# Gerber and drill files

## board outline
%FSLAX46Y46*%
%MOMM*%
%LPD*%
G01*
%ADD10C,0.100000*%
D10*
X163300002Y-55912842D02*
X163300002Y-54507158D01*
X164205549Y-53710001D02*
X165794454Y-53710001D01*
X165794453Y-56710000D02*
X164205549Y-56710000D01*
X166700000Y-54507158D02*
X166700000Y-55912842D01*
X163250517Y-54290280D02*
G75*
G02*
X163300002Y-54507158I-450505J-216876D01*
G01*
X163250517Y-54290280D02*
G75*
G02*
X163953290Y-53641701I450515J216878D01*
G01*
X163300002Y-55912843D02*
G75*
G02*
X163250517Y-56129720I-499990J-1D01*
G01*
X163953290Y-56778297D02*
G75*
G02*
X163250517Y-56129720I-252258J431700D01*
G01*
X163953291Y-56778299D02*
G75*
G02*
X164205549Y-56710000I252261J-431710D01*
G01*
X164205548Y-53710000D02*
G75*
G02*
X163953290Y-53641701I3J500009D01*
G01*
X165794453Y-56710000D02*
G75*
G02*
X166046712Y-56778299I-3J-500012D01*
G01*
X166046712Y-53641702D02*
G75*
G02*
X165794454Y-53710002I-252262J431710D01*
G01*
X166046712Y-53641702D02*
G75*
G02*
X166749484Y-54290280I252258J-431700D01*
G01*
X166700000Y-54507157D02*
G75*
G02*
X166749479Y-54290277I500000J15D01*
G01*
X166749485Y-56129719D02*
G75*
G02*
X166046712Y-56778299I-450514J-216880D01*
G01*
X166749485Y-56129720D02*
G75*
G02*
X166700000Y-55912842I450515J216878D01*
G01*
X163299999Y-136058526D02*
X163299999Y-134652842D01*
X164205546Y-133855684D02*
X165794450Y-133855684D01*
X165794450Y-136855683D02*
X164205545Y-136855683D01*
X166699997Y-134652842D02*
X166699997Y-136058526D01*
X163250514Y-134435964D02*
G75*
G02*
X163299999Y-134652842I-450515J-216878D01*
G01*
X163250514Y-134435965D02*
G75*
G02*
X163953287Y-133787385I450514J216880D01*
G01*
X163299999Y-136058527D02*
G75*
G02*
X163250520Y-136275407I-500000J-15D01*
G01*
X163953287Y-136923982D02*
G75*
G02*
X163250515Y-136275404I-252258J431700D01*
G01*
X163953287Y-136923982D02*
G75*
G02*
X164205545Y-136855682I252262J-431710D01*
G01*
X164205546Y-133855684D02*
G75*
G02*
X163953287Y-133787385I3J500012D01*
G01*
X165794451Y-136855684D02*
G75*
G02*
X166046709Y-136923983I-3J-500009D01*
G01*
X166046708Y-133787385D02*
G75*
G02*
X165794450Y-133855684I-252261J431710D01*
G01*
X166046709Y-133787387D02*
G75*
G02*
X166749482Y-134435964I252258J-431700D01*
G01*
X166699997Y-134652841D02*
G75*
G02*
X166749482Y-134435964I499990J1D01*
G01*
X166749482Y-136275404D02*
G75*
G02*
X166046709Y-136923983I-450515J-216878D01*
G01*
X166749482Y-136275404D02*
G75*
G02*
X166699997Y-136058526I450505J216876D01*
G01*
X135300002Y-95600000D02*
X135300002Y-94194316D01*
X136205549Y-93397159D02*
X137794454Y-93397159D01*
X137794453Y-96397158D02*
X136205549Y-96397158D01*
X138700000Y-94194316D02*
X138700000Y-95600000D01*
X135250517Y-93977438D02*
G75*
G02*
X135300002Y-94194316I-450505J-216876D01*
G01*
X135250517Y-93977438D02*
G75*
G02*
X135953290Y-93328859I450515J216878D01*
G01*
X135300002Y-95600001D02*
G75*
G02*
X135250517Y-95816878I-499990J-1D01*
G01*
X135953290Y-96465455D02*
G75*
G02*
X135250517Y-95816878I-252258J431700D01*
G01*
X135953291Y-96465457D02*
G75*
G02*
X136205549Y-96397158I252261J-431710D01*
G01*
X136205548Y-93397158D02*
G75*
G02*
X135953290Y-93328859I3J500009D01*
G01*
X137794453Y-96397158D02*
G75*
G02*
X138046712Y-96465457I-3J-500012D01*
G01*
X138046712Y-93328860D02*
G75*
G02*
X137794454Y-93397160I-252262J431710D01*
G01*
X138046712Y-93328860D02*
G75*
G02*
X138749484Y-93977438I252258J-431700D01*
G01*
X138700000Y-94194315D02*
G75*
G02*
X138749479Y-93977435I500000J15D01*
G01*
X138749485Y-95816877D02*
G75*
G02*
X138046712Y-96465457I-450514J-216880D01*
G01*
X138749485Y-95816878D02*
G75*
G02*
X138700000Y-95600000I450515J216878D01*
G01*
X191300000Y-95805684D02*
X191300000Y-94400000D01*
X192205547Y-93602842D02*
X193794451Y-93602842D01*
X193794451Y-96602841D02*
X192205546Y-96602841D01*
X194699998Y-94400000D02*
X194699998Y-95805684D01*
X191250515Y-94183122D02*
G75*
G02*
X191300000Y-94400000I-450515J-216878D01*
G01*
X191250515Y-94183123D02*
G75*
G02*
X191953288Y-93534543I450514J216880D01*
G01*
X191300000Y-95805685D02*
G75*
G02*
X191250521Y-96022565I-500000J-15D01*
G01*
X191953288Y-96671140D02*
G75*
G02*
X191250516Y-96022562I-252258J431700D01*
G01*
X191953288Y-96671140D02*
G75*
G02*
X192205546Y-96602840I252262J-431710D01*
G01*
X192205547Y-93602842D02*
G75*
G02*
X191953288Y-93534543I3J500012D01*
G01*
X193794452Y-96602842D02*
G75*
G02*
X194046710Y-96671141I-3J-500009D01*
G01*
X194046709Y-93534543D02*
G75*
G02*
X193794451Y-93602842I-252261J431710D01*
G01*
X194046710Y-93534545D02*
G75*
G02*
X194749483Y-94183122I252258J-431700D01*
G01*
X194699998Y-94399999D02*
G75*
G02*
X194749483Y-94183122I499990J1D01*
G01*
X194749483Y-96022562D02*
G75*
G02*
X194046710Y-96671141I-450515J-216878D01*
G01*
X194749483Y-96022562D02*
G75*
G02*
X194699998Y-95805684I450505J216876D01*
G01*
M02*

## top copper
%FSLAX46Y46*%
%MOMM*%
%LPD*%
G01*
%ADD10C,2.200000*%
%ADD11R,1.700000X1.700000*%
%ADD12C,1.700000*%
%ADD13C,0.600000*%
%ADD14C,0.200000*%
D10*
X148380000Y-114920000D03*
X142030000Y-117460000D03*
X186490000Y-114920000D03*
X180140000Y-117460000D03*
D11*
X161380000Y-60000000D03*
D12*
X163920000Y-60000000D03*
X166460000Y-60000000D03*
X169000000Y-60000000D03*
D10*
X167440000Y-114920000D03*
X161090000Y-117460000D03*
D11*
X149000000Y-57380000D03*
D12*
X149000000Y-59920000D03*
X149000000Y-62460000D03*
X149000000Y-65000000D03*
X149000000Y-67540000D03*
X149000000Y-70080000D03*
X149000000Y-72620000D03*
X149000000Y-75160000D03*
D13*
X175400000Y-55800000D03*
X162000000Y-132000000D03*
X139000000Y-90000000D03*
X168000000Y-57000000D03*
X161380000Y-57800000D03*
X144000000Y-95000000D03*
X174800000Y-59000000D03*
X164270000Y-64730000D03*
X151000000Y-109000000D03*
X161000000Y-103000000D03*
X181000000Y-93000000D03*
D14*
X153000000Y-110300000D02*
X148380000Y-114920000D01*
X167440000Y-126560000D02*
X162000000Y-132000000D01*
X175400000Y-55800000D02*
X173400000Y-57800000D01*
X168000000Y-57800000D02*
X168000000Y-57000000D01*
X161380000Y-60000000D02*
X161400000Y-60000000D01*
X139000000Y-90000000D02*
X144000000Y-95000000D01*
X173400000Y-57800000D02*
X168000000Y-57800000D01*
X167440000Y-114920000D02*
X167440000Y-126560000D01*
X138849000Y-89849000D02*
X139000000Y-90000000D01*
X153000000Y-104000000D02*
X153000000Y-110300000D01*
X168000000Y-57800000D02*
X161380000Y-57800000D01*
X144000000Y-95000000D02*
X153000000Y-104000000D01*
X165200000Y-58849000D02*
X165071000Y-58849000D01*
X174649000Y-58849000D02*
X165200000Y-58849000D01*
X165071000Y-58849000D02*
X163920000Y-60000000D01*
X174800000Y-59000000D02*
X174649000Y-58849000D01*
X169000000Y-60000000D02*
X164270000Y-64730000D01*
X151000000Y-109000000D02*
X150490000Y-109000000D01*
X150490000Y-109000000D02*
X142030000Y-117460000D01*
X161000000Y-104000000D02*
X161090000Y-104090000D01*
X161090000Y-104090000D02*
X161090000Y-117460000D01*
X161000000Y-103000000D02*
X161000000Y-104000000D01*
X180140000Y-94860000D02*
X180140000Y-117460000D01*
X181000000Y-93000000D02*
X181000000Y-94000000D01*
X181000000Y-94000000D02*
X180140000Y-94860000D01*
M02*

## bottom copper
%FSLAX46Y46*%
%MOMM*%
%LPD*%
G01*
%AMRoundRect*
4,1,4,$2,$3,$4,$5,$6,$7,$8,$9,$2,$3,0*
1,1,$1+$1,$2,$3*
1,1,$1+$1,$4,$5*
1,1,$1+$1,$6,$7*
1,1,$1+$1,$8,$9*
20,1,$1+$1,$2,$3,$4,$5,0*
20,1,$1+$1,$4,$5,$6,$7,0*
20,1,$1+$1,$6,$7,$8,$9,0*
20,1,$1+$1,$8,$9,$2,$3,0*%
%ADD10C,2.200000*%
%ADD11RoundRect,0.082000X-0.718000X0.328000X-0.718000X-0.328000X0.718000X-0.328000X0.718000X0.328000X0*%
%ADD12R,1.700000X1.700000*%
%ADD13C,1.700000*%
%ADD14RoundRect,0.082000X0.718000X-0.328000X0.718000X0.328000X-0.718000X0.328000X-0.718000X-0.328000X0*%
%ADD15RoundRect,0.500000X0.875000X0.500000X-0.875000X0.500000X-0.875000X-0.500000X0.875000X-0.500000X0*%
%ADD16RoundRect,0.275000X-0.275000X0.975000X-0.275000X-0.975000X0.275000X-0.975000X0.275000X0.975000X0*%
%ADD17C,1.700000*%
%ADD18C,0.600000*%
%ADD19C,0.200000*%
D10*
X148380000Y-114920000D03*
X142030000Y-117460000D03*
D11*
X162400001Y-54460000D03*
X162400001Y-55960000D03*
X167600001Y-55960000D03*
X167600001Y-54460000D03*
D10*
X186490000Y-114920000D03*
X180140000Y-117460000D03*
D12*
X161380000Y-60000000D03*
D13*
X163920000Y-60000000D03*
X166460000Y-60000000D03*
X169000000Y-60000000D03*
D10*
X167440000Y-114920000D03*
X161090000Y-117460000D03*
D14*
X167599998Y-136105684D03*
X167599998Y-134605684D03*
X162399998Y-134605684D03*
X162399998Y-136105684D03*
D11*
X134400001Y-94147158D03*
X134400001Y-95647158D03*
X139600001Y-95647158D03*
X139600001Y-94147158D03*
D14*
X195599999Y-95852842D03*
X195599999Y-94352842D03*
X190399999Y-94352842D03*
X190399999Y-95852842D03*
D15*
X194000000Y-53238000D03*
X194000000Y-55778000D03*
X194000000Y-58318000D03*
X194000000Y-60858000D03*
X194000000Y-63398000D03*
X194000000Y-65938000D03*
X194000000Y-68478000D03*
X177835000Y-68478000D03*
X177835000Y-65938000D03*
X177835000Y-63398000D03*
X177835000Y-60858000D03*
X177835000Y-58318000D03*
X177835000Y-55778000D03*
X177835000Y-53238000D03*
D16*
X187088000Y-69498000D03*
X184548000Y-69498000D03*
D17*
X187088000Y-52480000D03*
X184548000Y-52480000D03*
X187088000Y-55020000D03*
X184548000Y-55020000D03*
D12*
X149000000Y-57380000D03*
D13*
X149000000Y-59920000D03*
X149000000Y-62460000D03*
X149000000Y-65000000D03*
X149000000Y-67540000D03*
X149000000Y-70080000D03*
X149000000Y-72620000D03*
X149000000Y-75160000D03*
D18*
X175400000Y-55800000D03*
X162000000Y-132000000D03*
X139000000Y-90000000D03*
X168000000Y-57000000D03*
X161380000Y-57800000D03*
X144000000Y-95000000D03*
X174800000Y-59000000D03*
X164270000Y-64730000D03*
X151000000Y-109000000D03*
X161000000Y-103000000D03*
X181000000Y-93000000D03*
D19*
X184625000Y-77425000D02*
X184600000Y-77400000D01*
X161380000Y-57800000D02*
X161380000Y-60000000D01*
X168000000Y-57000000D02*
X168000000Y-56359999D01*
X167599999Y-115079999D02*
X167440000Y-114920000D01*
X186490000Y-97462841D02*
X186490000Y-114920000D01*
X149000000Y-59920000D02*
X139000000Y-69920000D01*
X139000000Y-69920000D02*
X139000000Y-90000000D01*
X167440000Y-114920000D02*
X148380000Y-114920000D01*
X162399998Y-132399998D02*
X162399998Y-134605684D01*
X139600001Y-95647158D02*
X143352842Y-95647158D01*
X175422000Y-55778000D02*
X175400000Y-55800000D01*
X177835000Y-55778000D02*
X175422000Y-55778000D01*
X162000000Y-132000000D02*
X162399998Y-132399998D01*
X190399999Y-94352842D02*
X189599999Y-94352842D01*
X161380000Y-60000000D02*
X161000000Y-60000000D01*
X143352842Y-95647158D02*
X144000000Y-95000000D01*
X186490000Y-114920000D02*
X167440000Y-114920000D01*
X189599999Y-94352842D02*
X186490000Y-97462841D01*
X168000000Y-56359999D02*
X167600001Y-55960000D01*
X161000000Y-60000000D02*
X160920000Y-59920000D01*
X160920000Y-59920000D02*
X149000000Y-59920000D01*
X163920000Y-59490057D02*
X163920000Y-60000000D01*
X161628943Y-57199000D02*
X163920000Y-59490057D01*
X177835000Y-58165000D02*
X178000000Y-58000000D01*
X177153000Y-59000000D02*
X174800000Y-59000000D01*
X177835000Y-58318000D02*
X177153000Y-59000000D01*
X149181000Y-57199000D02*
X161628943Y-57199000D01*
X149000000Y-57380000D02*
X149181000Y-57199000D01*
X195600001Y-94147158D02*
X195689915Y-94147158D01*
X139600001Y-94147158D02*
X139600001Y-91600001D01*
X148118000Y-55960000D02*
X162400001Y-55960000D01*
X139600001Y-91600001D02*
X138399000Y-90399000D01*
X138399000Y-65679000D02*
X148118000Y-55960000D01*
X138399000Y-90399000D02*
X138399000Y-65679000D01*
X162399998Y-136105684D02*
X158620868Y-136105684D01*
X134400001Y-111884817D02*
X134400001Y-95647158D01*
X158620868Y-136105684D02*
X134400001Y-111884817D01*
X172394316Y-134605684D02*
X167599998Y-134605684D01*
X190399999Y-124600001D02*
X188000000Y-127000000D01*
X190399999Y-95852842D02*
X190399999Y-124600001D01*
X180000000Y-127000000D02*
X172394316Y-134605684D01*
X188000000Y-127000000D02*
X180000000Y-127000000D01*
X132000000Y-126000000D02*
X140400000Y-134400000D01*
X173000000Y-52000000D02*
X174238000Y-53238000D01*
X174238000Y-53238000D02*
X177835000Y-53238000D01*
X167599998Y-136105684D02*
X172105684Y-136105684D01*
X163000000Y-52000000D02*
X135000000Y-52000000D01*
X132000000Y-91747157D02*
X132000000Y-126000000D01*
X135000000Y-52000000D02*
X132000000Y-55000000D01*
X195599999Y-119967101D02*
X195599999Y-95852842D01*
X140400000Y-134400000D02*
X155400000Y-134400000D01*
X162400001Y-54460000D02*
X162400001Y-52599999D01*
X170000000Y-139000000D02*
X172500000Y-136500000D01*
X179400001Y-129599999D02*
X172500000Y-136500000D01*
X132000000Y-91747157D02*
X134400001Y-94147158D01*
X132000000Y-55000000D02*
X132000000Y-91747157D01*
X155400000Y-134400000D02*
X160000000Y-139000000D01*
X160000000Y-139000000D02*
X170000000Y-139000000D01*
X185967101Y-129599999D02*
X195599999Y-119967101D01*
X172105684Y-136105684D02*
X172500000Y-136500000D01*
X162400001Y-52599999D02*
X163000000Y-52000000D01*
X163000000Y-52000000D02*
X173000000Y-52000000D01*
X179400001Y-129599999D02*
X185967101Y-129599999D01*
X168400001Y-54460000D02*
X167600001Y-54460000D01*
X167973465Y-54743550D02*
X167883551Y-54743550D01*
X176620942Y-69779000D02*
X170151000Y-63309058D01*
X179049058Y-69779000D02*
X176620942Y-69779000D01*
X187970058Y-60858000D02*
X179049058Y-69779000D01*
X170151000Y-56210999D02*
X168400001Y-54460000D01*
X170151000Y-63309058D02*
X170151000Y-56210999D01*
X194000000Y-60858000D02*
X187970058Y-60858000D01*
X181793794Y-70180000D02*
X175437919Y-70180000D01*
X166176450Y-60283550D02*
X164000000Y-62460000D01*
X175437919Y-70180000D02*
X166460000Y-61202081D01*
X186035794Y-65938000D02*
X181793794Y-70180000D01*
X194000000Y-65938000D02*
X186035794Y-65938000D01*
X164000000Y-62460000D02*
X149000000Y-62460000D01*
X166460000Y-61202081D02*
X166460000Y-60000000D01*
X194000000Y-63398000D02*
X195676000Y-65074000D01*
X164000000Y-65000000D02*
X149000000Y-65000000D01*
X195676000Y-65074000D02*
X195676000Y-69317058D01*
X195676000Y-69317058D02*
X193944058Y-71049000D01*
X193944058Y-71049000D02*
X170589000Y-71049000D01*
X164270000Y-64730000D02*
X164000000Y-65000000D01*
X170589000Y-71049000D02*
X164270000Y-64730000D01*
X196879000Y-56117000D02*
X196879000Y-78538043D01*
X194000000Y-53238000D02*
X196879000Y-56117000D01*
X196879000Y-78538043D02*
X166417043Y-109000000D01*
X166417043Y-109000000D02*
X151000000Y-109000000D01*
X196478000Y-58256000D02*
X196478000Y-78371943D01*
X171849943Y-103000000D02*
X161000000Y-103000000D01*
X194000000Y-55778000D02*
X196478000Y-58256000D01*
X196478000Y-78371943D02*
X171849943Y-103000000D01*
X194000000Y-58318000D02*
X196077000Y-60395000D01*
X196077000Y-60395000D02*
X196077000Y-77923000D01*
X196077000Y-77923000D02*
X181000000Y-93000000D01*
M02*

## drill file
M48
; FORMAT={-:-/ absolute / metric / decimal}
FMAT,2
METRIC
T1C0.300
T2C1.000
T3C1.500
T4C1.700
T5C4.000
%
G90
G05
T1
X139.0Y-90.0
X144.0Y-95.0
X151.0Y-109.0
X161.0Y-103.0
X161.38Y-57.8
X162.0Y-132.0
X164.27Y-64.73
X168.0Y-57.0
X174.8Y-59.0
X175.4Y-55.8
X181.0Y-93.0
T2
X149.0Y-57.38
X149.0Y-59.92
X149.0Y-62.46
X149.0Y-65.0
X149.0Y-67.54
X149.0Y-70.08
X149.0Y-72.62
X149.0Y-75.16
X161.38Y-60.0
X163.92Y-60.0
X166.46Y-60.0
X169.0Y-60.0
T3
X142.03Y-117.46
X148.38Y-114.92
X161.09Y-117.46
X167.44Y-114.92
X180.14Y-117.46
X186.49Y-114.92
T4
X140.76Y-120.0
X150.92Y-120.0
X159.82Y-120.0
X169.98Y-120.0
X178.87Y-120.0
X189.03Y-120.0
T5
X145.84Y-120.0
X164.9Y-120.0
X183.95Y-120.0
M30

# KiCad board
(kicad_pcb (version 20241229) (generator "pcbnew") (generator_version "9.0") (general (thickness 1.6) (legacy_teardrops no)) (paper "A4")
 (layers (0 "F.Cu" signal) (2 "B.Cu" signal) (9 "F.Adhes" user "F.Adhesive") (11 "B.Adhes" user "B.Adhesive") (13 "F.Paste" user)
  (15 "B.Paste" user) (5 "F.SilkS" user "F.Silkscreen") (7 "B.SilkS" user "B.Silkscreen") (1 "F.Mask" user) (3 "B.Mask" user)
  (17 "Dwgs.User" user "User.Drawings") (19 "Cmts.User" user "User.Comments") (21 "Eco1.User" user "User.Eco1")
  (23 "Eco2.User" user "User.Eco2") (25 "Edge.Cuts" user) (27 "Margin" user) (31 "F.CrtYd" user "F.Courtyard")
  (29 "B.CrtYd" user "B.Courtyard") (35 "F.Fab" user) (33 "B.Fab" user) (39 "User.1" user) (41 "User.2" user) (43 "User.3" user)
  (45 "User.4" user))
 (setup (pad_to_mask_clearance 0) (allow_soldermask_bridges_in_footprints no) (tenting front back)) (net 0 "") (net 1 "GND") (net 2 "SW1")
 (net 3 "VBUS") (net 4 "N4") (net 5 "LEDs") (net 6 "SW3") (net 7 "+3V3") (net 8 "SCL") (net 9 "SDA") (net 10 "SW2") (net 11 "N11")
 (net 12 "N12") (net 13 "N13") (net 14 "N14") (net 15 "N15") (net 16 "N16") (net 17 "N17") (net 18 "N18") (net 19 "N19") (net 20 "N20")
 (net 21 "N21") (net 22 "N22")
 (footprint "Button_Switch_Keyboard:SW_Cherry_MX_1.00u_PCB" (layer "F.Cu") (at 148.38 114.92)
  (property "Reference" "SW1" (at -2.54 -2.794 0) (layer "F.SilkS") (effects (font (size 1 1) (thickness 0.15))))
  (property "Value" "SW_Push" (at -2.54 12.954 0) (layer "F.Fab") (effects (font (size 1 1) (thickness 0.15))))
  (pad "" np_thru_hole circle (at -7.62 5.08) (size 1.7 1.7) (drill 1.7) (layers "*.Cu" "*.Mask"))
  (pad "" np_thru_hole circle (at -2.54 5.08) (size 4 4) (drill 4) (layers "*.Cu" "*.Mask"))
  (pad "" np_thru_hole circle (at 2.54 5.08) (size 1.7 1.7) (drill 1.7) (layers "*.Cu" "*.Mask"))
  (pad "1" thru_hole circle (at 0 0) (size 2.2 2.2) (drill 1.5) (layers "*.Cu" "*.Mask") (remove_unused_layers no) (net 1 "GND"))
  (pad "2" thru_hole circle (at -6.35 2.54) (size 2.2 2.2) (drill 1.5) (layers "*.Cu" "*.Mask") (remove_unused_layers no) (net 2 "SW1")))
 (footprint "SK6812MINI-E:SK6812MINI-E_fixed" (layer "F.Cu") (at 165 55.312842)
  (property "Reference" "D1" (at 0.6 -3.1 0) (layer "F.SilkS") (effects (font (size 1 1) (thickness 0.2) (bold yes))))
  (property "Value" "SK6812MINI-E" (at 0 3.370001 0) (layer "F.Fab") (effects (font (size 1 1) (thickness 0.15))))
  (fp_line (start -1.699998 0.6) (end -1.699998 -0.805684) (stroke (width 0.1) (type solid)) (layer "Edge.Cuts"))
  (fp_line (start -0.794451 -1.602841) (end 0.794454 -1.602841) (stroke (width 0.1) (type solid)) (layer "Edge.Cuts"))
  (fp_line (start 0.794453 1.397158) (end -0.794451 1.397158) (stroke (width 0.1) (type solid)) (layer "Edge.Cuts"))
  (fp_line (start 1.7 -0.805684) (end 1.7 0.6) (stroke (width 0.1) (type solid)) (layer "Edge.Cuts"))
  (fp_arc (start -1.749483 -1.022562) (mid -1.712526 -0.91691) (end -1.699998 -0.805684) (stroke (width 0.1) (type solid))
   (layer "Edge.Cuts"))
  (fp_arc (start -1.749483 -1.022562) (mid -1.63807 -1.606877) (end -1.04671 -1.671141) (stroke (width 0.1) (type solid))
   (layer "Edge.Cuts"))
  (fp_arc (start -1.699998 0.600001) (mid -1.712526 0.711226) (end -1.749483 0.816878) (stroke (width 0.1) (type solid)) (layer "Edge.Cuts"))
  (fp_arc (start -1.04671 1.465455) (mid -1.638069 1.401192) (end -1.749483 0.816878) (stroke (width 0.1) (type solid)) (layer "Edge.Cuts"))
  (fp_arc (start -1.046709 1.465457) (mid -0.925121 1.414535) (end -0.794451 1.397158) (stroke (width 0.1) (type solid)) (layer "Edge.Cuts"))
  (fp_arc (start -0.794452 -1.602842) (mid -0.925122 -1.620219) (end -1.04671 -1.671141) (stroke (width 0.1) (type solid))
   (layer "Edge.Cuts"))
  (fp_arc (start 0.794453 1.397158) (mid 0.925124 1.414535) (end 1.046712 1.465457) (stroke (width 0.1) (type solid)) (layer "Edge.Cuts"))
  (fp_arc (start 1.046712 -1.67114) (mid 0.925124 -1.620218) (end 0.794454 -1.602841) (stroke (width 0.1) (type solid)) (layer "Edge.Cuts"))
  (fp_arc (start 1.046712 -1.67114) (mid 1.638072 -1.606876) (end 1.749485 -1.022562) (stroke (width 0.1) (type solid)) (layer "Edge.Cuts"))
  (fp_arc (start 1.7 -0.805685) (mid 1.712528 -0.91691) (end 1.749485 -1.022562) (stroke (width 0.1) (type solid)) (layer "Edge.Cuts"))
  (fp_arc (start 1.749485 0.816877) (mid 1.638073 1.401193) (end 1.046712 1.465457) (stroke (width 0.1) (type solid)) (layer "Edge.Cuts"))
  (fp_arc (start 1.749485 0.816878) (mid 1.712528 0.711226) (end 1.7 0.6) (stroke (width 0.1) (type solid)) (layer "Edge.Cuts"))
  (pad "1" smd roundrect (at -2.599999 -0.852842 270) (size 0.82 1.6) (layers "B.Cu" "B.Mask" "B.Paste") (roundrect_rratio 0.1)
   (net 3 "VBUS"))
  (pad "2" smd roundrect (at -2.599999 0.647158 270) (size 0.82 1.6) (layers "B.Cu" "B.Mask" "B.Paste") (roundrect_rratio 0.1) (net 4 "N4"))
  (pad "3" smd roundrect (at 2.600001 0.647158 270) (size 0.82 1.6) (layers "B.Cu" "B.Mask" "B.Paste") (roundrect_rratio 0.1) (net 1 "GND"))
  (pad "4" smd roundrect (at 2.600001 -0.852842 270) (size 0.82 1.6) (layers "B.Cu" "B.Mask" "B.Paste") (roundrect_rratio 0.1)
   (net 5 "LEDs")))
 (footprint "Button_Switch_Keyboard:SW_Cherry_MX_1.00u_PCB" (layer "F.Cu") (at 186.49 114.92)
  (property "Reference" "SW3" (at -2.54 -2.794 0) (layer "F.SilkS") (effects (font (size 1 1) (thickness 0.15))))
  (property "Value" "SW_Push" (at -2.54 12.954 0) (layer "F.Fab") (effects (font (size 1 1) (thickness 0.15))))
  (pad "" np_thru_hole circle (at -7.62 5.08) (size 1.7 1.7) (drill 1.7) (layers "*.Cu" "*.Mask"))
  (pad "" np_thru_hole circle (at -2.54 5.08) (size 4 4) (drill 4) (layers "*.Cu" "*.Mask"))
  (pad "" np_thru_hole circle (at 2.54 5.08) (size 1.7 1.7) (drill 1.7) (layers "*.Cu" "*.Mask"))
  (pad "1" thru_hole circle (at 0 0) (size 2.2 2.2) (drill 1.5) (layers "*.Cu" "*.Mask") (remove_unused_layers no) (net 1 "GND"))
  (pad "2" thru_hole circle (at -6.35 2.54) (size 2.2 2.2) (drill 1.5) (layers "*.Cu" "*.Mask") (remove_unused_layers no) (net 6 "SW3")))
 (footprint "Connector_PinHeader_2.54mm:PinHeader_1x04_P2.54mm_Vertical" (layer "F.Cu") (at 161.38 60 90)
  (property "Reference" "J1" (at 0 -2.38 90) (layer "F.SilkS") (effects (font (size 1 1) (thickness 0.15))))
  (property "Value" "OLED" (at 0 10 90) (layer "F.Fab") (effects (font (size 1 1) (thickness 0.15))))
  (pad "1" thru_hole rect (at 0 0 90) (size 1.7 1.7) (drill 1) (layers "*.Cu" "*.Mask") (remove_unused_layers no) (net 1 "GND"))
  (pad "2" thru_hole circle (at 0 2.54 90) (size 1.7 1.7) (drill 1) (layers "*.Cu" "*.Mask") (remove_unused_layers no) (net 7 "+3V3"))
  (pad "3" thru_hole circle (at 0 5.08 90) (size 1.7 1.7) (drill 1) (layers "*.Cu" "*.Mask") (remove_unused_layers no) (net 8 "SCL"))
  (pad "4" thru_hole circle (at 0 7.62 90) (size 1.7 1.7) (drill 1) (layers "*.Cu" "*.Mask") (remove_unused_layers no) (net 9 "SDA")))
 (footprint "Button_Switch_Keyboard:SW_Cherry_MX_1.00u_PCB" (layer "F.Cu") (at 167.44 114.92)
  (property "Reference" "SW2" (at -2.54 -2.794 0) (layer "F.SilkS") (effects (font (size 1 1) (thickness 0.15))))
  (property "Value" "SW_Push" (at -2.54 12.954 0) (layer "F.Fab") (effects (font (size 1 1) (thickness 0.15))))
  (pad "" np_thru_hole circle (at -7.62 5.08) (size 1.7 1.7) (drill 1.7) (layers "*.Cu" "*.Mask"))
  (pad "" np_thru_hole circle (at -2.54 5.08) (size 4 4) (drill 4) (layers "*.Cu" "*.Mask"))
  (pad "" np_thru_hole circle (at 2.54 5.08) (size 1.7 1.7) (drill 1.7) (layers "*.Cu" "*.Mask"))
  (pad "1" thru_hole circle (at 0 0) (size 2.2 2.2) (drill 1.5) (layers "*.Cu" "*.Mask") (remove_unused_layers no) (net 1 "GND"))
  (pad "2" thru_hole circle (at -6.35 2.54) (size 2.2 2.2) (drill 1.5) (layers "*.Cu" "*.Mask") (remove_unused_layers no) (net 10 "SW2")))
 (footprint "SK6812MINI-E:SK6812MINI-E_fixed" (layer "F.Cu") (at 164.999999 135.252842 180)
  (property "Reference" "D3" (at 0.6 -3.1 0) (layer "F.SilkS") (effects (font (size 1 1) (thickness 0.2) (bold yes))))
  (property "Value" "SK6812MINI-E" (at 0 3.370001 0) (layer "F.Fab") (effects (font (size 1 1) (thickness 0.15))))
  (fp_line (start 1.7 -0.805684) (end 1.7 0.6) (stroke (width 0.1) (type solid)) (layer "Edge.Cuts"))
  (fp_line (start 0.794453 1.397158) (end -0.794451 1.397158) (stroke (width 0.1) (type solid)) (layer "Edge.Cuts"))
  (fp_line (start -0.794451 -1.602841) (end 0.794454 -1.602841) (stroke (width 0.1) (type solid)) (layer "Edge.Cuts"))
  (fp_line (start -1.699998 0.6) (end -1.699998 -0.805684) (stroke (width 0.1) (type solid)) (layer "Edge.Cuts"))
  (fp_arc (start 1.749485 0.816878) (mid 1.712528 0.711226) (end 1.7 0.6) (stroke (width 0.1) (type solid)) (layer "Edge.Cuts"))
  (fp_arc (start 1.749485 0.816877) (mid 1.638073 1.401193) (end 1.046712 1.465457) (stroke (width 0.1) (type solid)) (layer "Edge.Cuts"))
  (fp_arc (start 1.7 -0.805685) (mid 1.712528 -0.91691) (end 1.749485 -1.022562) (stroke (width 0.1) (type solid)) (layer "Edge.Cuts"))
  (fp_arc (start 1.046712 -1.67114) (mid 1.638072 -1.606876) (end 1.749485 -1.022562) (stroke (width 0.1) (type solid)) (layer "Edge.Cuts"))
  (fp_arc (start 1.046712 -1.67114) (mid 0.925124 -1.620218) (end 0.794454 -1.602841) (stroke (width 0.1) (type solid)) (layer "Edge.Cuts"))
  (fp_arc (start 0.794453 1.397158) (mid 0.925124 1.414535) (end 1.046712 1.465457) (stroke (width 0.1) (type solid)) (layer "Edge.Cuts"))
  (fp_arc (start -0.794452 -1.602842) (mid -0.925122 -1.620219) (end -1.04671 -1.671141) (stroke (width 0.1) (type solid))
   (layer "Edge.Cuts"))
  (fp_arc (start -1.046709 1.465457) (mid -0.925121 1.414535) (end -0.794451 1.397158) (stroke (width 0.1) (type solid)) (layer "Edge.Cuts"))
  (fp_arc (start -1.04671 1.465455) (mid -1.638069 1.401192) (end -1.749483 0.816878) (stroke (width 0.1) (type solid)) (layer "Edge.Cuts"))
  (fp_arc (start -1.699998 0.600001) (mid -1.712526 0.711226) (end -1.749483 0.816878) (stroke (width 0.1) (type solid)) (layer "Edge.Cuts"))
  (fp_arc (start -1.749483 -1.022562) (mid -1.63807 -1.606877) (end -1.04671 -1.671141) (stroke (width 0.1) (type solid))
   (layer "Edge.Cuts"))
  (fp_arc (start -1.749483 -1.022562) (mid -1.712526 -0.91691) (end -1.699998 -0.805684) (stroke (width 0.1) (type solid))
   (layer "Edge.Cuts"))
  (pad "1" smd roundrect (at -2.599999 -0.852842 90) (size 0.82 1.6) (layers "B.Cu" "B.Mask" "B.Paste") (roundrect_rratio 0.1)
   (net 3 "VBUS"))
  (pad "2" smd roundrect (at -2.599999 0.647158 90) (size 0.82 1.6) (layers "B.Cu" "B.Mask" "B.Paste") (roundrect_rratio 0.1) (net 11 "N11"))
  (pad "3" smd roundrect (at 2.600001 0.647158 90) (size 0.82 1.6) (layers "B.Cu" "B.Mask" "B.Paste") (roundrect_rratio 0.1) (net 1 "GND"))
  (pad "4" smd roundrect (at 2.600001 -0.852842 90) (size 0.82 1.6) (layers "B.Cu" "B.Mask" "B.Paste") (roundrect_rratio 0.1) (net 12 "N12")))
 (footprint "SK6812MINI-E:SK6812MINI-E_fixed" (layer "F.Cu") (at 137 95)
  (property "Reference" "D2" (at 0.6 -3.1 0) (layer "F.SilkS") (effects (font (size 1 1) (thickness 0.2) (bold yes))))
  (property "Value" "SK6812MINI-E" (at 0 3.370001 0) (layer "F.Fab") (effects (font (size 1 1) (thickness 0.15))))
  (fp_line (start -1.699998 0.6) (end -1.699998 -0.805684) (stroke (width 0.1) (type solid)) (layer "Edge.Cuts"))
  (fp_line (start -0.794451 -1.602841) (end 0.794454 -1.602841) (stroke (width 0.1) (type solid)) (layer "Edge.Cuts"))
  (fp_line (start 0.794453 1.397158) (end -0.794451 1.397158) (stroke (width 0.1) (type solid)) (layer "Edge.Cuts"))
  (fp_line (start 1.7 -0.805684) (end 1.7 0.6) (stroke (width 0.1) (type solid)) (layer "Edge.Cuts"))
  (fp_arc (start -1.749483 -1.022562) (mid -1.712526 -0.91691) (end -1.699998 -0.805684) (stroke (width 0.1) (type solid))
   (layer "Edge.Cuts"))
  (fp_arc (start -1.749483 -1.022562) (mid -1.63807 -1.606877) (end -1.04671 -1.671141) (stroke (width 0.1) (type solid))
   (layer "Edge.Cuts"))
  (fp_arc (start -1.699998 0.600001) (mid -1.712526 0.711226) (end -1.749483 0.816878) (stroke (width 0.1) (type solid)) (layer "Edge.Cuts"))
  (fp_arc (start -1.04671 1.465455) (mid -1.638069 1.401192) (end -1.749483 0.816878) (stroke (width 0.1) (type solid)) (layer "Edge.Cuts"))
  (fp_arc (start -1.046709 1.465457) (mid -0.925121 1.414535) (end -0.794451 1.397158) (stroke (width 0.1) (type solid)) (layer "Edge.Cuts"))
  (fp_arc (start -0.794452 -1.602842) (mid -0.925122 -1.620219) (end -1.04671 -1.671141) (stroke (width 0.1) (type solid))
   (layer "Edge.Cuts"))
  (fp_arc (start 0.794453 1.397158) (mid 0.925124 1.414535) (end 1.046712 1.465457) (stroke (width 0.1) (type solid)) (layer "Edge.Cuts"))
  (fp_arc (start 1.046712 -1.67114) (mid 0.925124 -1.620218) (end 0.794454 -1.602841) (stroke (width 0.1) (type solid)) (layer "Edge.Cuts"))
  (fp_arc (start 1.046712 -1.67114) (mid 1.638072 -1.606876) (end 1.749485 -1.022562) (stroke (width 0.1) (type solid)) (layer "Edge.Cuts"))
  (fp_arc (start 1.7 -0.805685) (mid 1.712528 -0.91691) (end 1.749485 -1.022562) (stroke (width 0.1) (type solid)) (layer "Edge.Cuts"))
  (fp_arc (start 1.749485 0.816877) (mid 1.638073 1.401193) (end 1.046712 1.465457) (stroke (width 0.1) (type solid)) (layer "Edge.Cuts"))
  (fp_arc (start 1.749485 0.816878) (mid 1.712528 0.711226) (end 1.7 0.6) (stroke (width 0.1) (type solid)) (layer "Edge.Cuts"))
  (pad "1" smd roundrect (at -2.599999 -0.852842 270) (size 0.82 1.6) (layers "B.Cu" "B.Mask" "B.Paste") (roundrect_rratio 0.1)
   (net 3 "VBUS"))
  (pad "2" smd roundrect (at -2.599999 0.647158 270) (size 0.82 1.6) (layers "B.Cu" "B.Mask" "B.Paste") (roundrect_rratio 0.1)
   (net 12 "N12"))
  (pad "3" smd roundrect (at 2.600001 0.647158 270) (size 0.82 1.6) (layers "B.Cu" "B.Mask" "B.Paste") (roundrect_rratio 0.1) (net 1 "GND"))
  (pad "4" smd roundrect (at 2.600001 -0.852842 270) (size 0.82 1.6) (layers "B.Cu" "B.Mask" "B.Paste") (roundrect_rratio 0.1) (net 4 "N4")))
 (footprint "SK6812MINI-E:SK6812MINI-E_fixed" (layer "F.Cu") (at 193 95 180)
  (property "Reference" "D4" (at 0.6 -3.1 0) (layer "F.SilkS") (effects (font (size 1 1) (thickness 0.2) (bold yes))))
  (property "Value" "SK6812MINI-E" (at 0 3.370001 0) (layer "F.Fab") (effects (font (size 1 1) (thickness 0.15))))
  (fp_line (start 1.7 -0.805684) (end 1.7 0.6) (stroke (width 0.1) (type solid)) (layer "Edge.Cuts"))
  (fp_line (start 0.794453 1.397158) (end -0.794451 1.397158) (stroke (width 0.1) (type solid)) (layer "Edge.Cuts"))
  (fp_line (start -0.794451 -1.602841) (end 0.794454 -1.602841) (stroke (width 0.1) (type solid)) (layer "Edge.Cuts"))
  (fp_line (start -1.699998 0.6) (end -1.699998 -0.805684) (stroke (width 0.1) (type solid)) (layer "Edge.Cuts"))
  (fp_arc (start 1.749485 0.816878) (mid 1.712528 0.711226) (end 1.7 0.6) (stroke (width 0.1) (type solid)) (layer "Edge.Cuts"))
  (fp_arc (start 1.749485 0.816877) (mid 1.638073 1.401193) (end 1.046712 1.465457) (stroke (width 0.1) (type solid)) (layer "Edge.Cuts"))
  (fp_arc (start 1.7 -0.805685) (mid 1.712528 -0.91691) (end 1.749485 -1.022562) (stroke (width 0.1) (type solid)) (layer "Edge.Cuts"))
  (fp_arc (start 1.046712 -1.67114) (mid 1.638072 -1.606876) (end 1.749485 -1.022562) (stroke (width 0.1) (type solid)) (layer "Edge.Cuts"))
  (fp_arc (start 1.046712 -1.67114) (mid 0.925124 -1.620218) (end 0.794454 -1.602841) (stroke (width 0.1) (type solid)) (layer "Edge.Cuts"))
  (fp_arc (start 0.794453 1.397158) (mid 0.925124 1.414535) (end 1.046712 1.465457) (stroke (width 0.1) (type solid)) (layer "Edge.Cuts"))
  (fp_arc (start -0.794452 -1.602842) (mid -0.925122 -1.620219) (end -1.04671 -1.671141) (stroke (width 0.1) (type solid))
   (layer "Edge.Cuts"))
  (fp_arc (start -1.046709 1.465457) (mid -0.925121 1.414535) (end -0.794451 1.397158) (stroke (width 0.1) (type solid)) (layer "Edge.Cuts"))
  (fp_arc (start -1.04671 1.465455) (mid -1.638069 1.401192) (end -1.749483 0.816878) (stroke (width 0.1) (type solid)) (layer "Edge.Cuts"))
  (fp_arc (start -1.699998 0.600001) (mid -1.712526 0.711226) (end -1.749483 0.816878) (stroke (width 0.1) (type solid)) (layer "Edge.Cuts"))
  (fp_arc (start -1.749483 -1.022562) (mid -1.63807 -1.606877) (end -1.04671 -1.671141) (stroke (width 0.1) (type solid))
   (layer "Edge.Cuts"))
  (fp_arc (start -1.749483 -1.022562) (mid -1.712526 -0.91691) (end -1.699998 -0.805684) (stroke (width 0.1) (type solid))
   (layer "Edge.Cuts"))
  (pad "1" smd roundrect (at -2.599999 -0.852842 90) (size 0.82 1.6) (layers "B.Cu" "B.Mask" "B.Paste") (roundrect_rratio 0.1)
   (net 3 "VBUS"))
  (pad "2" smd roundrect (at -2.599999 0.647158 90) (size 0.82 1.6) (layers "B.Cu" "B.Mask" "B.Paste") (roundrect_rratio 0.1) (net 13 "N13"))
  (pad "3" smd roundrect (at 2.600001 0.647158 90) (size 0.82 1.6) (layers "B.Cu" "B.Mask" "B.Paste") (roundrect_rratio 0.1) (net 1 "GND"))
  (pad "4" smd roundrect (at 2.600001 -0.852842 90) (size 0.82 1.6) (layers "B.Cu" "B.Mask" "B.Paste") (roundrect_rratio 0.1) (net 11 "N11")))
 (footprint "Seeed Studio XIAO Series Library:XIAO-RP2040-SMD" (layer "B.Cu") (at 186 60.858 180)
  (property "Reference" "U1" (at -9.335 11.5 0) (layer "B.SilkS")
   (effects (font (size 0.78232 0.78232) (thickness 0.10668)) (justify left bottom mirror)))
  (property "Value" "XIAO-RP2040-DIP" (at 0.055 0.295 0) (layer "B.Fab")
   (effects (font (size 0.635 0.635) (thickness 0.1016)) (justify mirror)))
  (pad "1" smd roundrect (at -8 7.62 180) (size 2.75 2) (layers "B.Cu" "B.Mask" "B.Paste") (roundrect_rratio 0.25) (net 2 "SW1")
   (solder_mask_margin 0.0508) (thermal_bridge_angle 45))
  (pad "2" smd roundrect (at -8 5.08 180) (size 2.75 2) (layers "B.Cu" "B.Mask" "B.Paste") (roundrect_rratio 0.25) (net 10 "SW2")
   (solder_mask_margin 0.0508) (thermal_bridge_angle 45))
  (pad "3" smd roundrect (at -8 2.54 180) (size 2.75 2) (layers "B.Cu" "B.Mask" "B.Paste") (roundrect_rratio 0.25) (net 6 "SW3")
   (solder_mask_margin 0.0508) (thermal_bridge_angle 45))
  (pad "4" smd roundrect (at -8 0 180) (size 2.75 2) (layers "B.Cu" "B.Mask" "B.Paste") (roundrect_rratio 0.25) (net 5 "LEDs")
   (solder_mask_margin 0.0508) (thermal_bridge_angle 45))
  (pad "5" smd roundrect (at -8 -2.54 180) (size 2.75 2) (layers "B.Cu" "B.Mask" "B.Paste") (roundrect_rratio 0.25) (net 9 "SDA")
   (solder_mask_margin 0.0508) (thermal_bridge_angle 45))
  (pad "6" smd roundrect (at -8 -5.08 180) (size 2.75 2) (layers "B.Cu" "B.Mask" "B.Paste") (roundrect_rratio 0.25) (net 8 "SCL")
   (solder_mask_margin 0.0508) (thermal_bridge_angle 45))
  (pad "7" smd roundrect (at -8 -7.62 180) (size 2.75 2) (layers "B.Cu" "B.Mask" "B.Paste") (roundrect_rratio 0.25) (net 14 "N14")
   (solder_mask_margin 0.0508) (thermal_bridge_angle 45))
  (pad "8" smd roundrect (at 8.165 -7.62 180) (size 2.75 2) (layers "B.Cu" "B.Mask" "B.Paste") (roundrect_rratio 0.25) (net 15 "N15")
   (solder_mask_margin 0.0508) (thermal_bridge_angle 45))
  (pad "9" smd roundrect (at 8.165 -5.08 180) (size 2.75 2) (layers "B.Cu" "B.Mask" "B.Paste") (roundrect_rratio 0.25) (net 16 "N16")
   (solder_mask_margin 0.0508) (thermal_bridge_angle 45))
  (pad "10" smd roundrect (at 8.165 -2.54 180) (size 2.75 2) (layers "B.Cu" "B.Mask" "B.Paste") (roundrect_rratio 0.25) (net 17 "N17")
   (solder_mask_margin 0.0508) (thermal_bridge_angle 45))
  (pad "11" smd roundrect (at 8.165 0 180) (size 2.75 2) (layers "B.Cu" "B.Mask" "B.Paste") (roundrect_rratio 0.25) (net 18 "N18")
   (solder_mask_margin 0.0508) (thermal_bridge_angle 45))
  (pad "12" smd roundrect (at 8.165 2.54 180) (size 2.75 2) (layers "B.Cu" "B.Mask" "B.Paste") (roundrect_rratio 0.25) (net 7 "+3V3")
   (solder_mask_margin 0.0508) (thermal_bridge_angle 45))
  (pad "13" smd roundrect (at 8.165 5.08 180) (size 2.75 2) (layers "B.Cu" "B.Mask" "B.Paste") (roundrect_rratio 0.25) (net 1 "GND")
   (solder_mask_margin 0.0508) (thermal_bridge_angle 45))
  (pad "14" smd roundrect (at 8.165 7.62 180) (size 2.75 2) (layers "B.Cu" "B.Mask" "B.Paste") (roundrect_rratio 0.25) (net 3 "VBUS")
   (solder_mask_margin 0.0508) (thermal_bridge_angle 45))
  (pad "15" smd roundrect (at -1.088 -8.64 270) (size 2.5 1.1) (layers "B.Cu" "B.Mask" "B.Paste") (roundrect_rratio 0.25)
   (thermal_bridge_angle 45))
  (pad "16" smd roundrect (at 1.452 -8.64 270) (size 2.5 1.1) (layers "B.Cu" "B.Mask" "B.Paste") (roundrect_rratio 0.25)
   (thermal_bridge_angle 45))
  (pad "17" smd circle (at -1.088 8.378 180) (size 1.7 1.7) (layers "B.Cu" "B.Mask" "B.Paste"))
  (pad "18" smd circle (at 1.452 8.378 180) (size 1.7 1.7) (layers "B.Cu" "B.Mask" "B.Paste"))
  (pad "19" smd circle (at -1.088 5.838 180) (size 1.7 1.7) (layers "B.Cu" "B.Mask" "B.Paste"))
  (pad "20" smd circle (at 1.452 5.838 180) (size 1.7 1.7) (layers "B.Cu" "B.Mask" "B.Paste")))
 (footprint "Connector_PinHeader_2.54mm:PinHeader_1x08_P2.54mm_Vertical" (layer "B.Cu") (at 149 57.38 180)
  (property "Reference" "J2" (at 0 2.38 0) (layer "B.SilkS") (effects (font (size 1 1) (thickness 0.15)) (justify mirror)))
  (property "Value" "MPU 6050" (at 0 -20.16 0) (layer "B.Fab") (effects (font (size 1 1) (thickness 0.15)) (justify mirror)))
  (pad "1" thru_hole rect (at 0 0 180) (size 1.7 1.7) (drill 1) (layers "*.Cu" "*.Mask") (remove_unused_layers no) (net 7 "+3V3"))
  (pad "2" thru_hole circle (at 0 -2.54 180) (size 1.7 1.7) (drill 1) (layers "*.Cu" "*.Mask") (remove_unused_layers no) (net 1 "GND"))
  (pad "3" thru_hole circle (at 0 -5.08 180) (size 1.7 1.7) (drill 1) (layers "*.Cu" "*.Mask") (remove_unused_layers no) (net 8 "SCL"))
  (pad "4" thru_hole circle (at 0 -7.62 180) (size 1.7 1.7) (drill 1) (layers "*.Cu" "*.Mask") (remove_unused_layers no) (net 9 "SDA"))
  (pad "5" thru_hole circle (at 0 -10.16 180) (size 1.7 1.7) (drill 1) (layers "*.Cu" "*.Mask") (remove_unused_layers no) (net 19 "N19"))
  (pad "6" thru_hole circle (at 0 -12.7 180) (size 1.7 1.7) (drill 1) (layers "*.Cu" "*.Mask") (remove_unused_layers no) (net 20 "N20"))
  (pad "7" thru_hole circle (at 0 -15.24 180) (size 1.7 1.7) (drill 1) (layers "*.Cu" "*.Mask") (remove_unused_layers no) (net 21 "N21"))
  (pad "8" thru_hole circle (at 0 -17.78 180) (size 1.7 1.7) (drill 1) (layers "*.Cu" "*.Mask") (remove_unused_layers no) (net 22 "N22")))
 (segment (start 184.625 77.425) (end 184.6 77.4) (width 0.2) (layer "B.Cu") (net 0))
 (segment (start 153 110.3) (end 148.38 114.92) (width 0.2) (layer "F.Cu") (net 1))
 (segment (start 167.44 126.56) (end 162 132) (width 0.2) (layer "F.Cu") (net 1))
 (segment (start 175.4 55.8) (end 173.4 57.8) (width 0.2) (layer "F.Cu") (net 1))
 (segment (start 168 57.8) (end 168 57) (width 0.2) (layer "F.Cu") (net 1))
 (segment (start 161.38 60) (end 161.4 60) (width 0.2) (layer "F.Cu") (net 1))
 (segment (start 139 90) (end 144 95) (width 0.2) (layer "F.Cu") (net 1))
 (segment (start 173.4 57.8) (end 168 57.8) (width 0.2) (layer "F.Cu") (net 1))
 (segment (start 167.44 114.92) (end 167.44 126.56) (width 0.2) (layer "F.Cu") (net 1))
 (segment (start 138.849 89.849) (end 139 90) (width 0.2) (layer "F.Cu") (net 1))
 (segment (start 153 104) (end 153 110.3) (width 0.2) (layer "F.Cu") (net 1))
 (segment (start 168 57.8) (end 161.38 57.8) (width 0.2) (layer "F.Cu") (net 1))
 (segment (start 144 95) (end 153 104) (width 0.2) (layer "F.Cu") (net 1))
 (via (at 175.4 55.8) (size 0.6) (drill 0.3) (layers "F.Cu" "B.Cu") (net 1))
 (via (at 162 132) (size 0.6) (drill 0.3) (layers "F.Cu" "B.Cu") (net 1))
 (via (at 139 90) (size 0.6) (drill 0.3) (layers "F.Cu" "B.Cu") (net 1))
 (via (at 168 57) (size 0.6) (drill 0.3) (layers "F.Cu" "B.Cu") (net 1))
 (via (at 161.38 57.8) (size 0.6) (drill 0.3) (layers "F.Cu" "B.Cu") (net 1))
 (via (at 144 95) (size 0.6) (drill 0.3) (layers "F.Cu" "B.Cu") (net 1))
 (segment (start 161.38 57.8) (end 161.38 60) (width 0.2) (layer "B.Cu") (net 1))
 (segment (start 168 57) (end 168 56.359999) (width 0.2) (layer "B.Cu") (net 1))
 (segment (start 167.599999 115.079999) (end 167.44 114.92) (width 0.2) (layer "B.Cu") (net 1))
 (segment (start 186.49 97.462841) (end 186.49 114.92) (width 0.2) (layer "B.Cu") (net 1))
 (segment (start 149 59.92) (end 139 69.92) (width 0.2) (layer "B.Cu") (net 1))
 (segment (start 139 69.92) (end 139 90) (width 0.2) (layer "B.Cu") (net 1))
 (segment (start 167.44 114.92) (end 148.38 114.92) (width 0.2) (layer "B.Cu") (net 1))
 (segment (start 162.399998 132.399998) (end 162.399998 134.605684) (width 0.2) (layer "B.Cu") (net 1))
 (segment (start 139.600001 95.647158) (end 143.352842 95.647158) (width 0.2) (layer "B.Cu") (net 1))
 (segment (start 175.422 55.778) (end 175.4 55.8) (width 0.2) (layer "B.Cu") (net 1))
 (segment (start 177.835 55.778) (end 175.422 55.778) (width 0.2) (layer "B.Cu") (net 1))
 (segment (start 162 132) (end 162.399998 132.399998) (width 0.2) (layer "B.Cu") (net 1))
 (segment (start 190.399999 94.352842) (end 189.599999 94.352842) (width 0.2) (layer "B.Cu") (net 1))
 (segment (start 161.38 60) (end 161 60) (width 0.2) (layer "B.Cu") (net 1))
 (segment (start 143.352842 95.647158) (end 144 95) (width 0.2) (layer "B.Cu") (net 1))
 (segment (start 186.49 114.92) (end 167.44 114.92) (width 0.2) (layer "B.Cu") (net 1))
 (segment (start 189.599999 94.352842) (end 186.49 97.462841) (width 0.2) (layer "B.Cu") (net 1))
 (segment (start 168 56.359999) (end 167.600001 55.96) (width 0.2) (layer "B.Cu") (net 1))
 (segment (start 161 60) (end 160.92 59.92) (width 0.2) (layer "B.Cu") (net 1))
 (segment (start 160.92 59.92) (end 149 59.92) (width 0.2) (layer "B.Cu") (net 1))
 (segment (start 165.2 58.849) (end 165.071 58.849) (width 0.2) (layer "F.Cu") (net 7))
 (segment (start 174.649 58.849) (end 165.2 58.849) (width 0.2) (layer "F.Cu") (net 7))
 (segment (start 165.071 58.849) (end 163.92 60) (width 0.2) (layer "F.Cu") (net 7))
 (segment (start 174.8 59) (end 174.649 58.849) (width 0.2) (layer "F.Cu") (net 7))
 (via (at 174.8 59) (size 0.6) (drill 0.3) (layers "F.Cu" "B.Cu") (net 7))
 (segment (start 163.92 59.490057) (end 163.92 60) (width 0.2) (layer "B.Cu") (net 7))
 (segment (start 161.628943 57.199) (end 163.92 59.490057) (width 0.2) (layer "B.Cu") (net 7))
 (segment (start 177.835 58.165) (end 178 58) (width 0.2) (layer "B.Cu") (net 7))
 (segment (start 177.153 59) (end 174.8 59) (width 0.2) (layer "B.Cu") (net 7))
 (segment (start 177.835 58.318) (end 177.153 59) (width 0.2) (layer "B.Cu") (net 7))
 (segment (start 149.181 57.199) (end 161.628943 57.199) (width 0.2) (layer "B.Cu") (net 7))
 (segment (start 149 57.38) (end 149.181 57.199) (width 0.2) (layer "B.Cu") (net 7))
 (segment (start 195.600001 94.147158) (end 195.689915 94.147158) (width 0.2) (layer "B.Cu") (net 13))
 (segment (start 139.600001 94.147158) (end 139.600001 91.600001) (width 0.2) (layer "B.Cu") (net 4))
 (segment (start 148.118 55.96) (end 162.400001 55.96) (width 0.2) (layer "B.Cu") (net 4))
 (segment (start 139.600001 91.600001) (end 138.399 90.399) (width 0.2) (layer "B.Cu") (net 4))
 (segment (start 138.399 65.679) (end 148.118 55.96) (width 0.2) (layer "B.Cu") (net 4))
 (segment (start 138.399 90.399) (end 138.399 65.679) (width 0.2) (layer "B.Cu") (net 4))
 (segment (start 162.399998 136.105684) (end 158.620868 136.105684) (width 0.2) (layer "B.Cu") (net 12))
 (segment (start 134.400001 111.884817) (end 134.400001 95.647158) (width 0.2) (layer "B.Cu") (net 12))
 (segment (start 158.620868 136.105684) (end 134.400001 111.884817) (width 0.2) (layer "B.Cu") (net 12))
 (segment (start 172.394316 134.605684) (end 167.599998 134.605684) (width 0.2) (layer "B.Cu") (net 11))
 (segment (start 190.399999 124.600001) (end 188 127) (width 0.2) (layer "B.Cu") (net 11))
 (segment (start 190.399999 95.852842) (end 190.399999 124.600001) (width 0.2) (layer "B.Cu") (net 11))
 (segment (start 180 127) (end 172.394316 134.605684) (width 0.2) (layer "B.Cu") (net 11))
 (segment (start 188 127) (end 180 127) (width 0.2) (layer "B.Cu") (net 11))
 (segment (start 132 126) (end 140.4 134.4) (width 0.2) (layer "B.Cu") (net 3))
 (segment (start 173 52) (end 174.238 53.238) (width 0.2) (layer "B.Cu") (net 3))
 (segment (start 174.238 53.238) (end 177.835 53.238) (width 0.2) (layer "B.Cu") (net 3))
 (segment (start 167.599998 136.105684) (end 172.105684 136.105684) (width 0.2) (layer "B.Cu") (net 3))
 (segment (start 163 52) (end 135 52) (width 0.2) (layer "B.Cu") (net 3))
 (segment (start 132 91.747157) (end 132 126) (width 0.2) (layer "B.Cu") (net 3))
 (segment (start 135 52) (end 132 55) (width 0.2) (layer "B.Cu") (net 3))
 (segment (start 195.599999 119.967101) (end 195.599999 95.852842) (width 0.2) (layer "B.Cu") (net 3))
 (segment (start 140.4 134.4) (end 155.4 134.4) (width 0.2) (layer "B.Cu") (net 3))
 (segment (start 162.400001 54.46) (end 162.400001 52.599999) (width 0.2) (layer "B.Cu") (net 3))
 (segment (start 170 139) (end 172.5 136.5) (width 0.2) (layer "B.Cu") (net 3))
 (segment (start 179.400001 129.599999) (end 172.5 136.5) (width 0.2) (layer "B.Cu") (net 3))
 (segment (start 132 91.747157) (end 134.400001 94.147158) (width 0.2) (layer "B.Cu") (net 3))
 (segment (start 132 55) (end 132 91.747157) (width 0.2) (layer "B.Cu") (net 3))
 (segment (start 155.4 134.4) (end 160 139) (width 0.2) (layer "B.Cu") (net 3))
 (segment (start 160 139) (end 170 139) (width 0.2) (layer "B.Cu") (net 3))
 (segment (start 185.967101 129.599999) (end 195.599999 119.967101) (width 0.2) (layer "B.Cu") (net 3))
 (segment (start 172.105684 136.105684) (end 172.5 136.5) (width 0.2) (layer "B.Cu") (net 3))
 (segment (start 162.400001 52.599999) (end 163 52) (width 0.2) (layer "B.Cu") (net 3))
 (segment (start 163 52) (end 173 52) (width 0.2) (layer "B.Cu") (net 3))
 (segment (start 179.400001 129.599999) (end 185.967101 129.599999) (width 0.2) (layer "B.Cu") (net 3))
 (segment (start 168.400001 54.46) (end 167.600001 54.46) (width 0.2) (layer "B.Cu") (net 5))
 (segment (start 167.973465 54.74355) (end 167.883551 54.74355) (width 0.2) (layer "B.Cu") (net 5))
 (segment (start 176.620942 69.779) (end 170.151 63.309058) (width 0.2) (layer "B.Cu") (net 5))
 (segment (start 179.049058 69.779) (end 176.620942 69.779) (width 0.2) (layer "B.Cu") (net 5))
 (segment (start 187.970058 60.858) (end 179.049058 69.779) (width 0.2) (layer "B.Cu") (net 5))
 (segment (start 170.151 56.210999) (end 168.400001 54.46) (width 0.2) (layer "B.Cu") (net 5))
 (segment (start 170.151 63.309058) (end 170.151 56.210999) (width 0.2) (layer "B.Cu") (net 5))
 (segment (start 194 60.858) (end 187.970058 60.858) (width 0.2) (layer "B.Cu") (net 5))
 (segment (start 181.793794 70.18) (end 175.437919 70.18) (width 0.2) (layer "B.Cu") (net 8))
 (segment (start 166.17645 60.28355) (end 164 62.46) (width 0.2) (layer "B.Cu") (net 8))
 (segment (start 175.437919 70.18) (end 166.46 61.202081) (width 0.2) (layer "B.Cu") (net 8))
 (segment (start 186.035794 65.938) (end 181.793794 70.18) (width 0.2) (layer "B.Cu") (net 8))
 (segment (start 194 65.938) (end 186.035794 65.938) (width 0.2) (layer "B.Cu") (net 8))
 (segment (start 164 62.46) (end 149 62.46) (width 0.2) (layer "B.Cu") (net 8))
 (segment (start 166.46 61.202081) (end 166.46 60) (width 0.2) (layer "B.Cu") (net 8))
 (segment (start 169 60) (end 164.27 64.73) (width 0.2) (layer "F.Cu") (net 9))
 (via (at 164.27 64.73) (size 0.6) (drill 0.3) (layers "F.Cu" "B.Cu") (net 9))
 (segment (start 194 63.398) (end 195.676 65.074) (width 0.2) (layer "B.Cu") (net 9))
 (segment (start 164 65) (end 149 65) (width 0.2) (layer "B.Cu") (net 9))
 (segment (start 195.676 65.074) (end 195.676 69.317058) (width 0.2) (layer "B.Cu") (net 9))
 (segment (start 195.676 69.317058) (end 193.944058 71.049) (width 0.2) (layer "B.Cu") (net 9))
 (segment (start 193.944058 71.049) (end 170.589 71.049) (width 0.2) (layer "B.Cu") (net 9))
 (segment (start 164.27 64.73) (end 164 65) (width 0.2) (layer "B.Cu") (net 9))
 (segment (start 170.589 71.049) (end 164.27 64.73) (width 0.2) (layer "B.Cu") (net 9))
 (segment (start 151 109) (end 150.49 109) (width 0.2) (layer "F.Cu") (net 2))
 (segment (start 150.49 109) (end 142.03 117.46) (width 0.2) (layer "F.Cu") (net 2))
 (via (at 151 109) (size 0.6) (drill 0.3) (layers "F.Cu" "B.Cu") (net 2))
 (segment (start 196.879 56.117) (end 196.879 78.538043) (width 0.2) (layer "B.Cu") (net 2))
 (segment (start 194 53.238) (end 196.879 56.117) (width 0.2) (layer "B.Cu") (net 2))
 (segment (start 196.879 78.538043) (end 166.417043 109) (width 0.2) (layer "B.Cu") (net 2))
 (segment (start 166.417043 109) (end 151 109) (width 0.2) (layer "B.Cu") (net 2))
 (segment (start 161 104) (end 161.09 104.09) (width 0.2) (layer "F.Cu") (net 10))
 (segment (start 161.09 104.09) (end 161.09 117.46) (width 0.2) (layer "F.Cu") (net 10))
 (segment (start 161 103) (end 161 104) (width 0.2) (layer "F.Cu") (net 10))
 (via (at 161 103) (size 0.6) (drill 0.3) (layers "F.Cu" "B.Cu") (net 10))
 (segment (start 196.478 58.256) (end 196.478 78.371943) (width 0.2) (layer "B.Cu") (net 10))
 (segment (start 171.849943 103) (end 161 103) (width 0.2) (layer "B.Cu") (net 10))
 (segment (start 194 55.778) (end 196.478 58.256) (width 0.2) (layer "B.Cu") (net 10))
 (segment (start 196.478 78.371943) (end 171.849943 103) (width 0.2) (layer "B.Cu") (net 10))
 (segment (start 180.14 94.86) (end 180.14 117.46) (width 0.2) (layer "F.Cu") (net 6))
 (segment (start 181 93) (end 181 94) (width 0.2) (layer "F.Cu") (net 6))
 (segment (start 181 94) (end 180.14 94.86) (width 0.2) (layer "F.Cu") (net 6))
 (via (at 181 93) (size 0.6) (drill 0.3) (layers "F.Cu" "B.Cu") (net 6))
 (segment (start 194 58.318) (end 196.077 60.395) (width 0.2) (layer "B.Cu") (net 6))
 (segment (start 196.077 60.395) (end 196.077 77.923) (width 0.2) (layer "B.Cu") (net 6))
 (segment (start 196.077 77.923) (end 181 93) (width 0.2) (layer "B.Cu") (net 6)))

